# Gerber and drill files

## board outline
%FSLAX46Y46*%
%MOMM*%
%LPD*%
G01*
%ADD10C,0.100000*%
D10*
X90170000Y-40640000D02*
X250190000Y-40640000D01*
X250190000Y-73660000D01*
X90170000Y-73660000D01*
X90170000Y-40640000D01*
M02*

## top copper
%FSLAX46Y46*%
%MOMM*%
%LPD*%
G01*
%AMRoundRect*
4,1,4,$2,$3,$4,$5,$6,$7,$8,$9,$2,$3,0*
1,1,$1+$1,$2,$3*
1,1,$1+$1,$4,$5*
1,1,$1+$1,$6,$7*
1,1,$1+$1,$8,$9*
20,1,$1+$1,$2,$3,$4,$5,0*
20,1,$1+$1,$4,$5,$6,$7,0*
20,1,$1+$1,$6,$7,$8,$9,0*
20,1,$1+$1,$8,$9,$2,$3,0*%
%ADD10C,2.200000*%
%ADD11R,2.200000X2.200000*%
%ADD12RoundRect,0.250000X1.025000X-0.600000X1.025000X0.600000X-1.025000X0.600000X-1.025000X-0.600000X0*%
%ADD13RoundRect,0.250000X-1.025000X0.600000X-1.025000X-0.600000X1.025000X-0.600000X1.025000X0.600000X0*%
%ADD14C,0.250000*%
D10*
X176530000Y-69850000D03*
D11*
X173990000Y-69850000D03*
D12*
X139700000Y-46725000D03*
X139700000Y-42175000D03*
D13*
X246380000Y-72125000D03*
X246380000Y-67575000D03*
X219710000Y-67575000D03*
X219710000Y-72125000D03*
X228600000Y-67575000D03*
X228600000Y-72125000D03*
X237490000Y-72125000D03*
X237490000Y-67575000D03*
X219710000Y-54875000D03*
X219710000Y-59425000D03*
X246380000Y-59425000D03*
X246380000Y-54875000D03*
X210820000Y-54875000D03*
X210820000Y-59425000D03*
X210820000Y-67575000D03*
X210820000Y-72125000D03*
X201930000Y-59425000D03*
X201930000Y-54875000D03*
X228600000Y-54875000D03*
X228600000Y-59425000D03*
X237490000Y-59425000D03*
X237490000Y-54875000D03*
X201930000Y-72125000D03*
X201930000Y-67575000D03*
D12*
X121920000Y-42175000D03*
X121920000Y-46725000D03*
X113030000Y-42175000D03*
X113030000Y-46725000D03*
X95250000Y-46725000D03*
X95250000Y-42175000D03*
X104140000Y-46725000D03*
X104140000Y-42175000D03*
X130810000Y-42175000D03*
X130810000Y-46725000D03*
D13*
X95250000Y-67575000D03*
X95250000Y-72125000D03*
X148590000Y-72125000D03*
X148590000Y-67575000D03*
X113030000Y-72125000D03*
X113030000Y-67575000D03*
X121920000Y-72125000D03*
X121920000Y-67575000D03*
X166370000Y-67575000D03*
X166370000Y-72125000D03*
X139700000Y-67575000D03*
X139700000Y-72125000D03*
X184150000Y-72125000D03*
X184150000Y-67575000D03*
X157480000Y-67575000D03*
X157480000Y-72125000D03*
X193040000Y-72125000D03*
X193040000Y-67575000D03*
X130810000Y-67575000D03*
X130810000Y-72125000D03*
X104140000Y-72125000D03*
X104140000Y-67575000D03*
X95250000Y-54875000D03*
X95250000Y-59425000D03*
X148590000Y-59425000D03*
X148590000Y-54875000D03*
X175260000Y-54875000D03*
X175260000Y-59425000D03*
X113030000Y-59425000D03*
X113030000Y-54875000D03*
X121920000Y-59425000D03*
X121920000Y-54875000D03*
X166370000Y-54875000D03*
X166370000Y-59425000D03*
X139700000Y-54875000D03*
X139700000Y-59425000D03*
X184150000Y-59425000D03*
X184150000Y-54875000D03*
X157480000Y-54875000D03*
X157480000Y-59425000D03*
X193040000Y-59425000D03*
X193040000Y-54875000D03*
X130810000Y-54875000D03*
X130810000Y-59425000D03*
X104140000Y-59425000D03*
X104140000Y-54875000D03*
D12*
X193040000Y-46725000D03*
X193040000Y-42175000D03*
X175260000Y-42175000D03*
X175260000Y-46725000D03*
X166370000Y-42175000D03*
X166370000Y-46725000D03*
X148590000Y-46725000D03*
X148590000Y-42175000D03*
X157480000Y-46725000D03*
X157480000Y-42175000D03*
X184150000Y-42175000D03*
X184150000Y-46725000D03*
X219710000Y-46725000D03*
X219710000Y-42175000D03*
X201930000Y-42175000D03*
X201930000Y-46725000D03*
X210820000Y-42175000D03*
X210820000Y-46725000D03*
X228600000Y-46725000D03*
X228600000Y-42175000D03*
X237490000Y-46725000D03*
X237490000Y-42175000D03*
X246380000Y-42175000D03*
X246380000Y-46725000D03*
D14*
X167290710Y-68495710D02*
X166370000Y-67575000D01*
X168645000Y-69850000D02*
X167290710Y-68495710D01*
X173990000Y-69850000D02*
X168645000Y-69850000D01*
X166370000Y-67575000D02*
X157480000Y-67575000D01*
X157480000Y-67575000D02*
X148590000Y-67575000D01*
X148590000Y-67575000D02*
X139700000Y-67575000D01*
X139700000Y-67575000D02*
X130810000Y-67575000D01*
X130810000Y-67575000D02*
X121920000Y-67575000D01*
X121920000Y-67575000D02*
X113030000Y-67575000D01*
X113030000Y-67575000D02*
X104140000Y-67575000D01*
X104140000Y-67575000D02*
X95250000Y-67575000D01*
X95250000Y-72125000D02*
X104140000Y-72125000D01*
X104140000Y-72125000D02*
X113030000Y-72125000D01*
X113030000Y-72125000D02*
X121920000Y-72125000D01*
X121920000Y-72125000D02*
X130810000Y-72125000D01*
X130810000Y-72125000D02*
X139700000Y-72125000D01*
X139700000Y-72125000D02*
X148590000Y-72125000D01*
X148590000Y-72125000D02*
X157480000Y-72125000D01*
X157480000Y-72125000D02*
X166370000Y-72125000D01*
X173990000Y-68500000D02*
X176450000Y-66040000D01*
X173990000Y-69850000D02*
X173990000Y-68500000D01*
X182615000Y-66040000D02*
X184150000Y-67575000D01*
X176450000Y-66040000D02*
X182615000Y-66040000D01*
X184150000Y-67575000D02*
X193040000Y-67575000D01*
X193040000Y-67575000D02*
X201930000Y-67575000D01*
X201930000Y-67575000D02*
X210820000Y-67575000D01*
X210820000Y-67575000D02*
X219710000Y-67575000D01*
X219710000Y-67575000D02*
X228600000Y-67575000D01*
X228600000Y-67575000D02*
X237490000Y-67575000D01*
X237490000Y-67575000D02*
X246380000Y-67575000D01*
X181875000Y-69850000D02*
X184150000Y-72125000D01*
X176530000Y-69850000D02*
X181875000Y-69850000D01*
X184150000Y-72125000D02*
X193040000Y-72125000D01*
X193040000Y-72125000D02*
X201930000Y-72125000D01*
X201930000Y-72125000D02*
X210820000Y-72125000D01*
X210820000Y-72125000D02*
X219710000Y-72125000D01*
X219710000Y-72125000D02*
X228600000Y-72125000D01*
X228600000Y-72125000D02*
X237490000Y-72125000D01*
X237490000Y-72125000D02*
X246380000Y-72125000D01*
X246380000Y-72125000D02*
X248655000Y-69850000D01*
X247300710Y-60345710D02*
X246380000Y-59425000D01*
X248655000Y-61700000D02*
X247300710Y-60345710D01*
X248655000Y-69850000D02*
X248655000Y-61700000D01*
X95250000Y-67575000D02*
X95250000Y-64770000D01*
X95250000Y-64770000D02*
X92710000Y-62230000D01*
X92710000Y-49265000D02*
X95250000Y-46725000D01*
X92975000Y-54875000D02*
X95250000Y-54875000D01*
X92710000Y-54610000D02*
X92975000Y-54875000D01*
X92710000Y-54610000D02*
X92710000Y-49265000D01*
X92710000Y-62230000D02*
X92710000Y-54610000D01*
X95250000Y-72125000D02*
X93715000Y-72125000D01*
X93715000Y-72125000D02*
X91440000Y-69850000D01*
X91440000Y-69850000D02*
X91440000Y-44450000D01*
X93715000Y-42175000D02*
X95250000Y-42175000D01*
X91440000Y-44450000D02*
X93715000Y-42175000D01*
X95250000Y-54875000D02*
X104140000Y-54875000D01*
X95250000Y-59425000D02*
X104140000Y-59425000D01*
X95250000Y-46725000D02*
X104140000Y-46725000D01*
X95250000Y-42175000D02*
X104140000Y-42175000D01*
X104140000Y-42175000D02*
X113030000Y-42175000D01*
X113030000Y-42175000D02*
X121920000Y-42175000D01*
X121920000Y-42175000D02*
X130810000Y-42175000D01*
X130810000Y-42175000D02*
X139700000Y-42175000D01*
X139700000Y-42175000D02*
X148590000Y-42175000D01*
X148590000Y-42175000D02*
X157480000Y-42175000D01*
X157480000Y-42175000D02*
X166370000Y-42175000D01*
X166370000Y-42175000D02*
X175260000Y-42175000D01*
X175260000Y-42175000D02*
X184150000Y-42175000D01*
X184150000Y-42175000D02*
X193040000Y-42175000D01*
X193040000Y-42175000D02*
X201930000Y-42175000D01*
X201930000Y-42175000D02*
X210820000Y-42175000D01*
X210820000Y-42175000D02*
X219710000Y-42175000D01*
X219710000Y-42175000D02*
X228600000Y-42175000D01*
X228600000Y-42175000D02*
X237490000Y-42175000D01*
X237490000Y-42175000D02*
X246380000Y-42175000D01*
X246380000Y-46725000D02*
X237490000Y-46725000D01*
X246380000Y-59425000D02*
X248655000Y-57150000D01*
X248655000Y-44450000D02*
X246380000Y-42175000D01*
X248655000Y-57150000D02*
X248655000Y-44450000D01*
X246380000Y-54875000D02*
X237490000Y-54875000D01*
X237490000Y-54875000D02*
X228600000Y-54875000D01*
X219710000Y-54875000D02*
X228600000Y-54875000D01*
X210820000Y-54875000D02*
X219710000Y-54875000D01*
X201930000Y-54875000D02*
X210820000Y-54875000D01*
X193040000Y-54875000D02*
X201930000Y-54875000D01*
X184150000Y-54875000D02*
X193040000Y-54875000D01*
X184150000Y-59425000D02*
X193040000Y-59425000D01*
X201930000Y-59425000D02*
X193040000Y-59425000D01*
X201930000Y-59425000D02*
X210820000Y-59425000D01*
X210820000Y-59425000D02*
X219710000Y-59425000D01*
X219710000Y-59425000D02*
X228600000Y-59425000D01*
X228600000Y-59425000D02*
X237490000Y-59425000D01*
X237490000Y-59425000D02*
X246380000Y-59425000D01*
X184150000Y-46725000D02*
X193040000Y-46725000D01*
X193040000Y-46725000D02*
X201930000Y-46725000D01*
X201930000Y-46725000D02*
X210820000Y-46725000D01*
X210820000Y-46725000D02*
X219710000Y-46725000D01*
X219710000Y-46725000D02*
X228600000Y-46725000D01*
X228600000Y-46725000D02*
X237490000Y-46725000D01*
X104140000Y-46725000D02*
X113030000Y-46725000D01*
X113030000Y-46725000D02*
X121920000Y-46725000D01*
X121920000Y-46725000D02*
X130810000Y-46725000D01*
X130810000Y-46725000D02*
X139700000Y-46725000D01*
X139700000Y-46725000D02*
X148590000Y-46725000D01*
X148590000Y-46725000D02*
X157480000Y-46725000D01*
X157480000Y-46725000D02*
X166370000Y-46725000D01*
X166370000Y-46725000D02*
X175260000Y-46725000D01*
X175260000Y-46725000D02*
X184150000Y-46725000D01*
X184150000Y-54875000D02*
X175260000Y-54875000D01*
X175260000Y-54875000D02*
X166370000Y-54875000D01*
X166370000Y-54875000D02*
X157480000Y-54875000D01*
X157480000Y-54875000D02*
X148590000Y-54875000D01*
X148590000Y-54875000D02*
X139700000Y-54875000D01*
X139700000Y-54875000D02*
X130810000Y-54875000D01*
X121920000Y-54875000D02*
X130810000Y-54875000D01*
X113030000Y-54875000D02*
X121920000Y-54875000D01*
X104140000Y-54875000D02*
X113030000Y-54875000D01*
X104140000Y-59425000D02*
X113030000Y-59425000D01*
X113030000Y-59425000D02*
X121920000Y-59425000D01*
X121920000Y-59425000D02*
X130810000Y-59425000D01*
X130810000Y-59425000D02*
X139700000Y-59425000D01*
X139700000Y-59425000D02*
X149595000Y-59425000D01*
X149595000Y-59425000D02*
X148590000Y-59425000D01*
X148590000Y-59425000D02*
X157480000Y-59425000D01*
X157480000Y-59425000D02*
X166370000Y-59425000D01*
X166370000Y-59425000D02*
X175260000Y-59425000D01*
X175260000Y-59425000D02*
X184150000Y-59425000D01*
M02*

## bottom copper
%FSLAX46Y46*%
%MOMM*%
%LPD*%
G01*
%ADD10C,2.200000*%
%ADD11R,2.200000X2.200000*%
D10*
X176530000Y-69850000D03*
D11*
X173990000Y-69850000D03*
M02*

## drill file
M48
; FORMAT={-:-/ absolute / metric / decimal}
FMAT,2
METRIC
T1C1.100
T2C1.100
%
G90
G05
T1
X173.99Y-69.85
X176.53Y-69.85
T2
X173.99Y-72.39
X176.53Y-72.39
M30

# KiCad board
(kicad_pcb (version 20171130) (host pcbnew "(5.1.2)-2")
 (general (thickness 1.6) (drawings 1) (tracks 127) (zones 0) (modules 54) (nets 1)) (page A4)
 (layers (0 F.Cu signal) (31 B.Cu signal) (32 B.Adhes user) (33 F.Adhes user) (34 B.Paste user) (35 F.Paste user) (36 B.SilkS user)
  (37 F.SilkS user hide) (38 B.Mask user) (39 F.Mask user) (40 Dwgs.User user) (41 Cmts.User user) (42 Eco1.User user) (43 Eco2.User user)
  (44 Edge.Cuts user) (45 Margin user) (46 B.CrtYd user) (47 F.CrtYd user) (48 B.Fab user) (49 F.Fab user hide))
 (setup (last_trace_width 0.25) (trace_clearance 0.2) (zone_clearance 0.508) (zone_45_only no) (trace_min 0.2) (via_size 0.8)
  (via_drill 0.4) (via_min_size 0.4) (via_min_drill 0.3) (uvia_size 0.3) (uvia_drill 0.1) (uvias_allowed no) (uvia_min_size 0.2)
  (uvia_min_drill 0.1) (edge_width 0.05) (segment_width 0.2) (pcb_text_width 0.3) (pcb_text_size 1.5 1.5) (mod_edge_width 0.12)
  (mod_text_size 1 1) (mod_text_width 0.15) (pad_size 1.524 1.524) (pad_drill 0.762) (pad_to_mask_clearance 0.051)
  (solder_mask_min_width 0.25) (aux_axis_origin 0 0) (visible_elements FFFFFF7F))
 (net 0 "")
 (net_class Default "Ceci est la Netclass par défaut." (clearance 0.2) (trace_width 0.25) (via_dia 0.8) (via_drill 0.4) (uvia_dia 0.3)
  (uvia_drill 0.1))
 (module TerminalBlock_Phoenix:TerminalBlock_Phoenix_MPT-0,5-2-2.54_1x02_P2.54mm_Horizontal (layer F.Cu) (at 173.99 69.85)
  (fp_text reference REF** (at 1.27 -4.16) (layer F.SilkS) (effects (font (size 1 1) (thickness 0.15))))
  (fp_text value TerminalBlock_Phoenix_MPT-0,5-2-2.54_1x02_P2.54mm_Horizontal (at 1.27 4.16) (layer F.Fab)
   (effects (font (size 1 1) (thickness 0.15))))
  (pad "" np_thru_hole circle (at 2.54 2.54) (size 1.1 1.1) (drill 1.1) (layers *.Cu *.Mask))
  (pad 2 thru_hole circle (at 2.54 0) (size 2.2 2.2) (drill 1.1) (layers *.Cu *.Mask))
  (pad "" np_thru_hole circle (at 0 2.54) (size 1.1 1.1) (drill 1.1) (layers *.Cu *.Mask))
  (pad 1 thru_hole rect (at 0 0) (size 2.2 2.2) (drill 1.1) (layers *.Cu *.Mask)))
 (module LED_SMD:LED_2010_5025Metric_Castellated (layer F.Cu) (at 139.7 44.45 90)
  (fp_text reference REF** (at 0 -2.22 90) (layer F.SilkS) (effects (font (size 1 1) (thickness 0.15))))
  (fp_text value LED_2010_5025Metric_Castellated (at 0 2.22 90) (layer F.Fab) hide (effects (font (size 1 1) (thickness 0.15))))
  (pad 1 smd roundrect (at -2.275 0 90) (size 1.7 2.55) (layers F.Cu F.Paste F.Mask) (roundrect_rratio 0.147059))
  (pad 2 smd roundrect (at 2.275 0 90) (size 1.7 2.55) (layers F.Cu F.Paste F.Mask) (roundrect_rratio 0.147059)))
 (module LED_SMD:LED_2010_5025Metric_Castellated (layer F.Cu) (at 246.38 69.85 270)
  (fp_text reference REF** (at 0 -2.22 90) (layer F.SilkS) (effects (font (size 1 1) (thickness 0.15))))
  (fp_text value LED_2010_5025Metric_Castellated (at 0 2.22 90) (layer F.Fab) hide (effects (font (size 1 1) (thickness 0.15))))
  (pad 2 smd roundrect (at 2.275 0 270) (size 1.7 2.55) (layers F.Cu F.Paste F.Mask) (roundrect_rratio 0.147059))
  (pad 1 smd roundrect (at -2.275 0 270) (size 1.7 2.55) (layers F.Cu F.Paste F.Mask) (roundrect_rratio 0.147059)))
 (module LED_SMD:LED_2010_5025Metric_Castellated (layer F.Cu) (at 219.71 69.85 270)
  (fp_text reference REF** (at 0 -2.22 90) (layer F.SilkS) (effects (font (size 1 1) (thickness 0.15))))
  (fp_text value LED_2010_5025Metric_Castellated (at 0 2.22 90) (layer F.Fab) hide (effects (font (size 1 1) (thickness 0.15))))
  (pad 1 smd roundrect (at -2.275 0 270) (size 1.7 2.55) (layers F.Cu F.Paste F.Mask) (roundrect_rratio 0.147059))
  (pad 2 smd roundrect (at 2.275 0 270) (size 1.7 2.55) (layers F.Cu F.Paste F.Mask) (roundrect_rratio 0.147059)))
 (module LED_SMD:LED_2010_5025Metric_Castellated (layer F.Cu) (at 228.6 69.85 270)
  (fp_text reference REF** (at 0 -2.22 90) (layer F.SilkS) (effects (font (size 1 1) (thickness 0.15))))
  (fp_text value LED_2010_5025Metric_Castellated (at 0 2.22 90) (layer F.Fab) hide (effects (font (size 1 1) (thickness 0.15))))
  (pad 1 smd roundrect (at -2.275 0 270) (size 1.7 2.55) (layers F.Cu F.Paste F.Mask) (roundrect_rratio 0.147059))
  (pad 2 smd roundrect (at 2.275 0 270) (size 1.7 2.55) (layers F.Cu F.Paste F.Mask) (roundrect_rratio 0.147059)))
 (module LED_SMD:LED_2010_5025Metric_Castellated (layer F.Cu) (at 237.49 69.85 270)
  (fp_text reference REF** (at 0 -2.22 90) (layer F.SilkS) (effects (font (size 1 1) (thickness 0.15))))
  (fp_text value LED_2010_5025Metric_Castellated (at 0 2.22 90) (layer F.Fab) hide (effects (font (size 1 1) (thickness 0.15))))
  (pad 2 smd roundrect (at 2.275 0 270) (size 1.7 2.55) (layers F.Cu F.Paste F.Mask) (roundrect_rratio 0.147059))
  (pad 1 smd roundrect (at -2.275 0 270) (size 1.7 2.55) (layers F.Cu F.Paste F.Mask) (roundrect_rratio 0.147059)))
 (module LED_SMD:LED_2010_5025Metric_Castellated (layer F.Cu) (at 219.71 57.15 270)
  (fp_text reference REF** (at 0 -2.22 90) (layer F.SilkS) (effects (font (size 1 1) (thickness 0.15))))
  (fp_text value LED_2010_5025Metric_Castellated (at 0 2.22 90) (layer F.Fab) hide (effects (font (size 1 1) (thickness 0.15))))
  (pad 1 smd roundrect (at -2.275 0 270) (size 1.7 2.55) (layers F.Cu F.Paste F.Mask) (roundrect_rratio 0.147059))
  (pad 2 smd roundrect (at 2.275 0 270) (size 1.7 2.55) (layers F.Cu F.Paste F.Mask) (roundrect_rratio 0.147059)))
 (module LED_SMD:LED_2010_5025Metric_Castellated (layer F.Cu) (at 246.38 57.15 270)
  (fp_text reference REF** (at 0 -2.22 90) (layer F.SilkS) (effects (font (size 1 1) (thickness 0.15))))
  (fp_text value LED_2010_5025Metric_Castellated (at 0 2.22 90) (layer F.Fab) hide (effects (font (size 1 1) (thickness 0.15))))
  (pad 2 smd roundrect (at 2.275 0 270) (size 1.7 2.55) (layers F.Cu F.Paste F.Mask) (roundrect_rratio 0.147059))
  (pad 1 smd roundrect (at -2.275 0 270) (size 1.7 2.55) (layers F.Cu F.Paste F.Mask) (roundrect_rratio 0.147059)))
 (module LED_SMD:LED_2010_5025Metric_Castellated (layer F.Cu) (at 210.82 57.15 270)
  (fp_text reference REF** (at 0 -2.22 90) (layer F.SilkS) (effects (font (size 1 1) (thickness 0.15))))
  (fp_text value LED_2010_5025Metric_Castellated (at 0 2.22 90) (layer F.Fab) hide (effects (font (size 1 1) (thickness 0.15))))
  (pad 1 smd roundrect (at -2.275 0 270) (size 1.7 2.55) (layers F.Cu F.Paste F.Mask) (roundrect_rratio 0.147059))
  (pad 2 smd roundrect (at 2.275 0 270) (size 1.7 2.55) (layers F.Cu F.Paste F.Mask) (roundrect_rratio 0.147059)))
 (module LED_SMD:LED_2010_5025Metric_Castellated (layer F.Cu) (at 210.82 69.85 270)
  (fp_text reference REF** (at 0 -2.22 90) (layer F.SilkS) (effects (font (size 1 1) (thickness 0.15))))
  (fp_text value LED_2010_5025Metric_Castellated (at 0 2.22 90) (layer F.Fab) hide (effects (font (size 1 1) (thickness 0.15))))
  (pad 1 smd roundrect (at -2.275 0 270) (size 1.7 2.55) (layers F.Cu F.Paste F.Mask) (roundrect_rratio 0.147059))
  (pad 2 smd roundrect (at 2.275 0 270) (size 1.7 2.55) (layers F.Cu F.Paste F.Mask) (roundrect_rratio 0.147059)))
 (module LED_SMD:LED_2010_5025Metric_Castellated (layer F.Cu) (at 201.93 57.15 270)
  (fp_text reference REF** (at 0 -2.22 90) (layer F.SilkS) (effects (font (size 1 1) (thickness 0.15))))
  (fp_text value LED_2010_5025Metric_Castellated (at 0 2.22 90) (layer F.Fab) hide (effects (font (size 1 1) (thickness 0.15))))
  (pad 2 smd roundrect (at 2.275 0 270) (size 1.7 2.55) (layers F.Cu F.Paste F.Mask) (roundrect_rratio 0.147059))
  (pad 1 smd roundrect (at -2.275 0 270) (size 1.7 2.55) (layers F.Cu F.Paste F.Mask) (roundrect_rratio 0.147059)))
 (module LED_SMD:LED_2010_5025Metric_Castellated (layer F.Cu) (at 228.6 57.15 270)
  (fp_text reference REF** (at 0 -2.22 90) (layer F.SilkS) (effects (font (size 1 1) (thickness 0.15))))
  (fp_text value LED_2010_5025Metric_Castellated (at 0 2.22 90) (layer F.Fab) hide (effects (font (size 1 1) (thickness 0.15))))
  (pad 1 smd roundrect (at -2.275 0 270) (size 1.7 2.55) (layers F.Cu F.Paste F.Mask) (roundrect_rratio 0.147059))
  (pad 2 smd roundrect (at 2.275 0 270) (size 1.7 2.55) (layers F.Cu F.Paste F.Mask) (roundrect_rratio 0.147059)))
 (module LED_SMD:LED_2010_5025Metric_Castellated (layer F.Cu) (at 237.49 57.15 270)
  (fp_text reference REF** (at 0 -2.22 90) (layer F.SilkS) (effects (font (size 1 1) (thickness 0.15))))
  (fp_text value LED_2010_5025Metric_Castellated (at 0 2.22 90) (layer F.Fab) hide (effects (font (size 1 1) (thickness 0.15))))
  (pad 2 smd roundrect (at 2.275 0 270) (size 1.7 2.55) (layers F.Cu F.Paste F.Mask) (roundrect_rratio 0.147059))
  (pad 1 smd roundrect (at -2.275 0 270) (size 1.7 2.55) (layers F.Cu F.Paste F.Mask) (roundrect_rratio 0.147059)))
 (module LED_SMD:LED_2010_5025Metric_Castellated (layer F.Cu) (at 201.93 69.85 270)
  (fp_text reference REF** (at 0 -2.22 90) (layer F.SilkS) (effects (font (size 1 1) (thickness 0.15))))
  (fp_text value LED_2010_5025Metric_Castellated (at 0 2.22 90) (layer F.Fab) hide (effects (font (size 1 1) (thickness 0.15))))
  (pad 2 smd roundrect (at 2.275 0 270) (size 1.7 2.55) (layers F.Cu F.Paste F.Mask) (roundrect_rratio 0.147059))
  (pad 1 smd roundrect (at -2.275 0 270) (size 1.7 2.55) (layers F.Cu F.Paste F.Mask) (roundrect_rratio 0.147059)))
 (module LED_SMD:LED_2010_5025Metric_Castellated (layer F.Cu) (at 121.92 44.45 90)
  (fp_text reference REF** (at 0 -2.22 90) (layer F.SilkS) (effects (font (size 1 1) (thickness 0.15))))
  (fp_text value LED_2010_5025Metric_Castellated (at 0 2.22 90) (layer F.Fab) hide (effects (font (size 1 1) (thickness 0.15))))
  (pad 2 smd roundrect (at 2.275 0 90) (size 1.7 2.55) (layers F.Cu F.Paste F.Mask) (roundrect_rratio 0.147059))
  (pad 1 smd roundrect (at -2.275 0 90) (size 1.7 2.55) (layers F.Cu F.Paste F.Mask) (roundrect_rratio 0.147059)))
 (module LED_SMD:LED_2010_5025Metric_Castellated (layer F.Cu) (at 113.03 44.45 90)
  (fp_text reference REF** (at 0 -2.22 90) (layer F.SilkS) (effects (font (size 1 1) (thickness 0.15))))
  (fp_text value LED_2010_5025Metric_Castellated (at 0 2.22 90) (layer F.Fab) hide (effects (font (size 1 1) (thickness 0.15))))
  (pad 2 smd roundrect (at 2.275 0 90) (size 1.7 2.55) (layers F.Cu F.Paste F.Mask) (roundrect_rratio 0.147059))
  (pad 1 smd roundrect (at -2.275 0 90) (size 1.7 2.55) (layers F.Cu F.Paste F.Mask) (roundrect_rratio 0.147059)))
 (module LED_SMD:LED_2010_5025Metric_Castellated (layer F.Cu) (at 95.25 44.45 90)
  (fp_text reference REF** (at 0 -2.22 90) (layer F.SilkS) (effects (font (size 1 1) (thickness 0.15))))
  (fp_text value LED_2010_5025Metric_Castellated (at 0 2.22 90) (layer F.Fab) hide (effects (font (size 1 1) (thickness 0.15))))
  (pad 1 smd roundrect (at -2.275 0 90) (size 1.7 2.55) (layers F.Cu F.Paste F.Mask) (roundrect_rratio 0.147059))
  (pad 2 smd roundrect (at 2.275 0 90) (size 1.7 2.55) (layers F.Cu F.Paste F.Mask) (roundrect_rratio 0.147059)))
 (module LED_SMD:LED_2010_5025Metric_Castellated (layer F.Cu) (at 104.14 44.45 90)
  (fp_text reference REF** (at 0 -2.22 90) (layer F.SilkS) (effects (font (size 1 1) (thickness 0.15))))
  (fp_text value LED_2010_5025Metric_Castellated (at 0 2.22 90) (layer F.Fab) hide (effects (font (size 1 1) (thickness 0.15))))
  (pad 1 smd roundrect (at -2.275 0 90) (size 1.7 2.55) (layers F.Cu F.Paste F.Mask) (roundrect_rratio 0.147059))
  (pad 2 smd roundrect (at 2.275 0 90) (size 1.7 2.55) (layers F.Cu F.Paste F.Mask) (roundrect_rratio 0.147059)))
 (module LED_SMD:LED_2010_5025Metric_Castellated (layer F.Cu) (at 130.81 44.45 90)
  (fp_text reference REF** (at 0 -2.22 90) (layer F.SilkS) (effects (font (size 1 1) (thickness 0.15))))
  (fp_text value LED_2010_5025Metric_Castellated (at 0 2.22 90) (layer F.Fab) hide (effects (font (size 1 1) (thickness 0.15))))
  (pad 2 smd roundrect (at 2.275 0 90) (size 1.7 2.55) (layers F.Cu F.Paste F.Mask) (roundrect_rratio 0.147059))
  (pad 1 smd roundrect (at -2.275 0 90) (size 1.7 2.55) (layers F.Cu F.Paste F.Mask) (roundrect_rratio 0.147059)))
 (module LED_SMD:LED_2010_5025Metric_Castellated (layer F.Cu) (at 95.25 69.85 270)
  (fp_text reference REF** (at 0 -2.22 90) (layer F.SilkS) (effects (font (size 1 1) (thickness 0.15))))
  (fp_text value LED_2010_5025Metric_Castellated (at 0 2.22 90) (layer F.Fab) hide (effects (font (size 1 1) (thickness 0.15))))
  (pad 1 smd roundrect (at -2.275 0 270) (size 1.7 2.55) (layers F.Cu F.Paste F.Mask) (roundrect_rratio 0.147059))
  (pad 2 smd roundrect (at 2.275 0 270) (size 1.7 2.55) (layers F.Cu F.Paste F.Mask) (roundrect_rratio 0.147059)))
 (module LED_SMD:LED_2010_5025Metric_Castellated (layer F.Cu) (at 148.59 69.85 270)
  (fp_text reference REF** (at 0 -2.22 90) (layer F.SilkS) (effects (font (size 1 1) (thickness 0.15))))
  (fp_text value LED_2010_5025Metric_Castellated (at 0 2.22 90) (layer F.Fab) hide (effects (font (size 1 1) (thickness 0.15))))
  (pad 2 smd roundrect (at 2.275 0 270) (size 1.7 2.55) (layers F.Cu F.Paste F.Mask) (roundrect_rratio 0.147059))
  (pad 1 smd roundrect (at -2.275 0 270) (size 1.7 2.55) (layers F.Cu F.Paste F.Mask) (roundrect_rratio 0.147059)))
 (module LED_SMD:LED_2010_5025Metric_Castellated (layer F.Cu) (at 113.03 69.85 270)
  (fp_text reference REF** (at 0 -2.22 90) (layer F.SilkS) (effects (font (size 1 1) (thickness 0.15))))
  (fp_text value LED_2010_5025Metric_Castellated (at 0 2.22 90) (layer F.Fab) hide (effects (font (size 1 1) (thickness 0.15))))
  (pad 2 smd roundrect (at 2.275 0 270) (size 1.7 2.55) (layers F.Cu F.Paste F.Mask) (roundrect_rratio 0.147059))
  (pad 1 smd roundrect (at -2.275 0 270) (size 1.7 2.55) (layers F.Cu F.Paste F.Mask) (roundrect_rratio 0.147059)))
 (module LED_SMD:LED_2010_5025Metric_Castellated (layer F.Cu) (at 121.92 69.85 270)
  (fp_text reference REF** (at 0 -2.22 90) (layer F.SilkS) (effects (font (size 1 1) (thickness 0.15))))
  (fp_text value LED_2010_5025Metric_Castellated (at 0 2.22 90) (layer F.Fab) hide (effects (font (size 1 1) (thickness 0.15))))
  (pad 2 smd roundrect (at 2.275 0 270) (size 1.7 2.55) (layers F.Cu F.Paste F.Mask) (roundrect_rratio 0.147059))
  (pad 1 smd roundrect (at -2.275 0 270) (size 1.7 2.55) (layers F.Cu F.Paste F.Mask) (roundrect_rratio 0.147059)))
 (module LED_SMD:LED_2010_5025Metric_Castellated (layer F.Cu) (at 166.37 69.85 270)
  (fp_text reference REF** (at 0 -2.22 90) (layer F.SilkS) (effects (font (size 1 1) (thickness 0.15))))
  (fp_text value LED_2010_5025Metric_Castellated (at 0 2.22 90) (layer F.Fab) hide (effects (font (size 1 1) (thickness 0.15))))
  (pad 1 smd roundrect (at -2.275 0 270) (size 1.7 2.55) (layers F.Cu F.Paste F.Mask) (roundrect_rratio 0.147059))
  (pad 2 smd roundrect (at 2.275 0 270) (size 1.7 2.55) (layers F.Cu F.Paste F.Mask) (roundrect_rratio 0.147059)))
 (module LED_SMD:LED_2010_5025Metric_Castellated (layer F.Cu) (at 139.7 69.85 270)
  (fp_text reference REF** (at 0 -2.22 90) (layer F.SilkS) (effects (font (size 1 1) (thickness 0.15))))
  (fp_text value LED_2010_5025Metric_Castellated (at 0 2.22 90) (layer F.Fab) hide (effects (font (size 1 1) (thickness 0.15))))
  (pad 1 smd roundrect (at -2.275 0 270) (size 1.7 2.55) (layers F.Cu F.Paste F.Mask) (roundrect_rratio 0.147059))
  (pad 2 smd roundrect (at 2.275 0 270) (size 1.7 2.55) (layers F.Cu F.Paste F.Mask) (roundrect_rratio 0.147059)))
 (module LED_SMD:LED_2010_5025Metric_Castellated (layer F.Cu) (at 184.15 69.85 270)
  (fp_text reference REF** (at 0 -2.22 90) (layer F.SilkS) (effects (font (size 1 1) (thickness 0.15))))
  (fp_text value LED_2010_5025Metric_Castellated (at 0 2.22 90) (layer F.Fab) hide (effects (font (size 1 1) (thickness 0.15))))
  (pad 2 smd roundrect (at 2.275 0 270) (size 1.7 2.55) (layers F.Cu F.Paste F.Mask) (roundrect_rratio 0.147059))
  (pad 1 smd roundrect (at -2.275 0 270) (size 1.7 2.55) (layers F.Cu F.Paste F.Mask) (roundrect_rratio 0.147059)))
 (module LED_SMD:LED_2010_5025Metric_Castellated (layer F.Cu) (at 157.48 69.85 270)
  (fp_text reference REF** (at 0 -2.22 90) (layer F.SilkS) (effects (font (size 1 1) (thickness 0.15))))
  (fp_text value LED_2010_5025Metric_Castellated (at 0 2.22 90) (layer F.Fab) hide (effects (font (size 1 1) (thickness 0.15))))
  (pad 1 smd roundrect (at -2.275 0 270) (size 1.7 2.55) (layers F.Cu F.Paste F.Mask) (roundrect_rratio 0.147059))
  (pad 2 smd roundrect (at 2.275 0 270) (size 1.7 2.55) (layers F.Cu F.Paste F.Mask) (roundrect_rratio 0.147059)))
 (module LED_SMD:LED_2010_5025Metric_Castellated (layer F.Cu) (at 193.04 69.85 270)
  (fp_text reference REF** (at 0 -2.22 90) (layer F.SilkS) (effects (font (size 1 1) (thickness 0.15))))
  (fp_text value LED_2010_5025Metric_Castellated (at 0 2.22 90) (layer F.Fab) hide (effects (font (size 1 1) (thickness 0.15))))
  (pad 2 smd roundrect (at 2.275 0 270) (size 1.7 2.55) (layers F.Cu F.Paste F.Mask) (roundrect_rratio 0.147059))
  (pad 1 smd roundrect (at -2.275 0 270) (size 1.7 2.55) (layers F.Cu F.Paste F.Mask) (roundrect_rratio 0.147059)))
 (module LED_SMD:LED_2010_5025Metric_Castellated (layer F.Cu) (at 130.81 69.85 270)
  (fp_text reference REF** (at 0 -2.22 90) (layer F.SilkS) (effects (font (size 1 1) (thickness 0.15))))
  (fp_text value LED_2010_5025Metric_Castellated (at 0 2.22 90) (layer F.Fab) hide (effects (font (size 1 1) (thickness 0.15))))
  (pad 1 smd roundrect (at -2.275 0 270) (size 1.7 2.55) (layers F.Cu F.Paste F.Mask) (roundrect_rratio 0.147059))
  (pad 2 smd roundrect (at 2.275 0 270) (size 1.7 2.55) (layers F.Cu F.Paste F.Mask) (roundrect_rratio 0.147059)))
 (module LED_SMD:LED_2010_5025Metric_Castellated (layer F.Cu) (at 104.14 69.85 270)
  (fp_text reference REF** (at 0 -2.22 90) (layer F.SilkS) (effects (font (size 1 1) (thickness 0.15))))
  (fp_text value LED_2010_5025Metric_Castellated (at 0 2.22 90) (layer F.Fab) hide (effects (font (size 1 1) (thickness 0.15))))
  (pad 2 smd roundrect (at 2.275 0 270) (size 1.7 2.55) (layers F.Cu F.Paste F.Mask) (roundrect_rratio 0.147059))
  (pad 1 smd roundrect (at -2.275 0 270) (size 1.7 2.55) (layers F.Cu F.Paste F.Mask) (roundrect_rratio 0.147059)))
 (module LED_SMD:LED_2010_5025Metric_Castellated (layer F.Cu) (at 95.25 57.15 270)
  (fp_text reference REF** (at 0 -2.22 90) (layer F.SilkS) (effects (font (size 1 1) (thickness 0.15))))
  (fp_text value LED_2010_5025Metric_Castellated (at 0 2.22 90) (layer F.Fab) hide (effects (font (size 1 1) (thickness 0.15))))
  (pad 1 smd roundrect (at -2.275 0 270) (size 1.7 2.55) (layers F.Cu F.Paste F.Mask) (roundrect_rratio 0.147059))
  (pad 2 smd roundrect (at 2.275 0 270) (size 1.7 2.55) (layers F.Cu F.Paste F.Mask) (roundrect_rratio 0.147059)))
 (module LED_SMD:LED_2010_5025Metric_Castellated (layer F.Cu) (at 148.59 57.15 270)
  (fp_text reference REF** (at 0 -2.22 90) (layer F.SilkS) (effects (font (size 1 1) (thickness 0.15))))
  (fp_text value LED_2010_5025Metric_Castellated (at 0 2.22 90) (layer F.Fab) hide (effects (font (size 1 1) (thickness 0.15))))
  (pad 2 smd roundrect (at 2.275 0 270) (size 1.7 2.55) (layers F.Cu F.Paste F.Mask) (roundrect_rratio 0.147059))
  (pad 1 smd roundrect (at -2.275 0 270) (size 1.7 2.55) (layers F.Cu F.Paste F.Mask) (roundrect_rratio 0.147059)))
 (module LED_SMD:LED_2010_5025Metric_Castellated (layer F.Cu) (at 175.26 57.15 270)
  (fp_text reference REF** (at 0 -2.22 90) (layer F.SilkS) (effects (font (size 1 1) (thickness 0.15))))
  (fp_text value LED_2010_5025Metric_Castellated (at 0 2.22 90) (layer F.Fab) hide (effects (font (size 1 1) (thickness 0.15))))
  (pad 1 smd roundrect (at -2.275 0 270) (size 1.7 2.55) (layers F.Cu F.Paste F.Mask) (roundrect_rratio 0.147059))
  (pad 2 smd roundrect (at 2.275 0 270) (size 1.7 2.55) (layers F.Cu F.Paste F.Mask) (roundrect_rratio 0.147059)))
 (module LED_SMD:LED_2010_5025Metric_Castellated (layer F.Cu) (at 113.03 57.15 270)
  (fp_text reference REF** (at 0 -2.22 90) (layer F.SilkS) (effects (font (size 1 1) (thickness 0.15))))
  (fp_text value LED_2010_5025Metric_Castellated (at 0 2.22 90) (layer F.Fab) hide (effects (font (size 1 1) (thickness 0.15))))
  (pad 2 smd roundrect (at 2.275 0 270) (size 1.7 2.55) (layers F.Cu F.Paste F.Mask) (roundrect_rratio 0.147059))
  (pad 1 smd roundrect (at -2.275 0 270) (size 1.7 2.55) (layers F.Cu F.Paste F.Mask) (roundrect_rratio 0.147059)))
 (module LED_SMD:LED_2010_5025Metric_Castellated (layer F.Cu) (at 121.92 57.15 270)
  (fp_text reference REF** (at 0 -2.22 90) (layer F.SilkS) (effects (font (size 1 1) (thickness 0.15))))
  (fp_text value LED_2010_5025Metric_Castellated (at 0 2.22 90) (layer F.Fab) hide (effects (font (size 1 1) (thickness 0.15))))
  (pad 2 smd roundrect (at 2.275 0 270) (size 1.7 2.55) (layers F.Cu F.Paste F.Mask) (roundrect_rratio 0.147059))
  (pad 1 smd roundrect (at -2.275 0 270) (size 1.7 2.55) (layers F.Cu F.Paste F.Mask) (roundrect_rratio 0.147059)))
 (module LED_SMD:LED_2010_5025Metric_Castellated (layer F.Cu) (at 166.37 57.15 270)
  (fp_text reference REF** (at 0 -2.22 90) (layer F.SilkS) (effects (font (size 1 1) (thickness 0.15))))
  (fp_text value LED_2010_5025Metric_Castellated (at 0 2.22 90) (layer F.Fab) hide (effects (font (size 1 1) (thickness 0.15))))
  (pad 1 smd roundrect (at -2.275 0 270) (size 1.7 2.55) (layers F.Cu F.Paste F.Mask) (roundrect_rratio 0.147059))
  (pad 2 smd roundrect (at 2.275 0 270) (size 1.7 2.55) (layers F.Cu F.Paste F.Mask) (roundrect_rratio 0.147059)))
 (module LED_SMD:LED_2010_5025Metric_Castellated (layer F.Cu) (at 139.7 57.15 270)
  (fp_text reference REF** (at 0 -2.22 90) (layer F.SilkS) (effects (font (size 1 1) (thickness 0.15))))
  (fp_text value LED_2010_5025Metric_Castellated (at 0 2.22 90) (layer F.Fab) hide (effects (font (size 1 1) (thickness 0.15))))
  (pad 1 smd roundrect (at -2.275 0 270) (size 1.7 2.55) (layers F.Cu F.Paste F.Mask) (roundrect_rratio 0.147059))
  (pad 2 smd roundrect (at 2.275 0 270) (size 1.7 2.55) (layers F.Cu F.Paste F.Mask) (roundrect_rratio 0.147059)))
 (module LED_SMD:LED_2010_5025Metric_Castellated (layer F.Cu) (at 184.15 57.15 270)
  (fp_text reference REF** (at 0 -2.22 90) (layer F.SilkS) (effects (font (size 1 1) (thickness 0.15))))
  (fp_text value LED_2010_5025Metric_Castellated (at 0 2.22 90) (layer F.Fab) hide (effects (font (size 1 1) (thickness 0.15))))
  (pad 2 smd roundrect (at 2.275 0 270) (size 1.7 2.55) (layers F.Cu F.Paste F.Mask) (roundrect_rratio 0.147059))
  (pad 1 smd roundrect (at -2.275 0 270) (size 1.7 2.55) (layers F.Cu F.Paste F.Mask) (roundrect_rratio 0.147059)))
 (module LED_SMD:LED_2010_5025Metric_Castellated (layer F.Cu) (at 157.48 57.15 270)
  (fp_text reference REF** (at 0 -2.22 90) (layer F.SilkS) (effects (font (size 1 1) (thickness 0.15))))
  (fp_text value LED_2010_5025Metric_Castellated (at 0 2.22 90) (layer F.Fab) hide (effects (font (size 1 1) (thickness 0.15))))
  (pad 1 smd roundrect (at -2.275 0 270) (size 1.7 2.55) (layers F.Cu F.Paste F.Mask) (roundrect_rratio 0.147059))
  (pad 2 smd roundrect (at 2.275 0 270) (size 1.7 2.55) (layers F.Cu F.Paste F.Mask) (roundrect_rratio 0.147059)))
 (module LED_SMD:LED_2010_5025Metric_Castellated (layer F.Cu) (at 193.04 57.15 270)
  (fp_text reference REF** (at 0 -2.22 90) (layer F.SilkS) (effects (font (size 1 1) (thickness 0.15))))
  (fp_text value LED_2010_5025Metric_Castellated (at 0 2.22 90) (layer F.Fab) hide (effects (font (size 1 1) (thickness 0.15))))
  (pad 2 smd roundrect (at 2.275 0 270) (size 1.7 2.55) (layers F.Cu F.Paste F.Mask) (roundrect_rratio 0.147059))
  (pad 1 smd roundrect (at -2.275 0 270) (size 1.7 2.55) (layers F.Cu F.Paste F.Mask) (roundrect_rratio 0.147059)))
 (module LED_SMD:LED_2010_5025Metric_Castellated (layer F.Cu) (at 130.81 57.15 270)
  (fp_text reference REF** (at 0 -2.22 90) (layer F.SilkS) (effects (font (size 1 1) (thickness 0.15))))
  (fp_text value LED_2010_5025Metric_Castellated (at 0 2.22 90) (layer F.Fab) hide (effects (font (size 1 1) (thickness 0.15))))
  (pad 1 smd roundrect (at -2.275 0 270) (size 1.7 2.55) (layers F.Cu F.Paste F.Mask) (roundrect_rratio 0.147059))
  (pad 2 smd roundrect (at 2.275 0 270) (size 1.7 2.55) (layers F.Cu F.Paste F.Mask) (roundrect_rratio 0.147059)))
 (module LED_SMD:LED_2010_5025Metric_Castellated (layer F.Cu) (at 104.14 57.15 270)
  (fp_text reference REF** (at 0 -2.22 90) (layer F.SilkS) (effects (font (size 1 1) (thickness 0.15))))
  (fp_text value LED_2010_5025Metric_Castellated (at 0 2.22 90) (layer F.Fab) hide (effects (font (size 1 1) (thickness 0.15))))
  (pad 2 smd roundrect (at 2.275 0 270) (size 1.7 2.55) (layers F.Cu F.Paste F.Mask) (roundrect_rratio 0.147059))
  (pad 1 smd roundrect (at -2.275 0 270) (size 1.7 2.55) (layers F.Cu F.Paste F.Mask) (roundrect_rratio 0.147059)))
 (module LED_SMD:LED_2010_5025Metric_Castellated (layer F.Cu) (at 193.04 44.45 90)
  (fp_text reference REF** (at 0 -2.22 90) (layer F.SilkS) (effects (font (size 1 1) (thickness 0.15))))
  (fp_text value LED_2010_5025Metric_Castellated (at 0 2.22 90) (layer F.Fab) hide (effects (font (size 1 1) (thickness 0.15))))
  (pad 1 smd roundrect (at -2.275 0 90) (size 1.7 2.55) (layers F.Cu F.Paste F.Mask) (roundrect_rratio 0.147059))
  (pad 2 smd roundrect (at 2.275 0 90) (size 1.7 2.55) (layers F.Cu F.Paste F.Mask) (roundrect_rratio 0.147059)))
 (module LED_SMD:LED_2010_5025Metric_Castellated (layer F.Cu) (at 175.26 44.45 90)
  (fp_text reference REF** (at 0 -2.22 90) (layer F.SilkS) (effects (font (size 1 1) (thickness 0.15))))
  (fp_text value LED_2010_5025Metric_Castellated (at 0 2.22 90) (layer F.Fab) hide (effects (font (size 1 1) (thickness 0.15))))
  (pad 2 smd roundrect (at 2.275 0 90) (size 1.7 2.55) (layers F.Cu F.Paste F.Mask) (roundrect_rratio 0.147059))
  (pad 1 smd roundrect (at -2.275 0 90) (size 1.7 2.55) (layers F.Cu F.Paste F.Mask) (roundrect_rratio 0.147059)))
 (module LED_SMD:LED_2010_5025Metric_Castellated (layer F.Cu) (at 166.37 44.45 90)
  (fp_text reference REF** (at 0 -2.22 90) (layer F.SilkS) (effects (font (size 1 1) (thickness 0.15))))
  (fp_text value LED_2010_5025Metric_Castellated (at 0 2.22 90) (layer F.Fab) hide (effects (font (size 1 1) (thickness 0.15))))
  (pad 2 smd roundrect (at 2.275 0 90) (size 1.7 2.55) (layers F.Cu F.Paste F.Mask) (roundrect_rratio 0.147059))
  (pad 1 smd roundrect (at -2.275 0 90) (size 1.7 2.55) (layers F.Cu F.Paste F.Mask) (roundrect_rratio 0.147059)))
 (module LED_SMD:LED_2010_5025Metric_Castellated (layer F.Cu) (at 148.59 44.45 90)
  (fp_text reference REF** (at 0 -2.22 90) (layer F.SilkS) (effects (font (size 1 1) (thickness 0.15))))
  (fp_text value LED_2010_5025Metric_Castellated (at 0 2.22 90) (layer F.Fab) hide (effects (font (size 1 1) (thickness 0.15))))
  (pad 1 smd roundrect (at -2.275 0 90) (size 1.7 2.55) (layers F.Cu F.Paste F.Mask) (roundrect_rratio 0.147059))
  (pad 2 smd roundrect (at 2.275 0 90) (size 1.7 2.55) (layers F.Cu F.Paste F.Mask) (roundrect_rratio 0.147059)))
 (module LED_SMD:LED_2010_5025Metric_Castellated (layer F.Cu) (at 157.48 44.45 90)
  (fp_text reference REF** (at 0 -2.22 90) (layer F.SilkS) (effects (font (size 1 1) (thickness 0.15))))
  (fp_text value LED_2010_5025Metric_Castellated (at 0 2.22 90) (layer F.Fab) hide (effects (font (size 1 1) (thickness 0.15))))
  (pad 1 smd roundrect (at -2.275 0 90) (size 1.7 2.55) (layers F.Cu F.Paste F.Mask) (roundrect_rratio 0.147059))
  (pad 2 smd roundrect (at 2.275 0 90) (size 1.7 2.55) (layers F.Cu F.Paste F.Mask) (roundrect_rratio 0.147059)))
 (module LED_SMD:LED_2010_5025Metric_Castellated (layer F.Cu) (at 184.15 44.45 90)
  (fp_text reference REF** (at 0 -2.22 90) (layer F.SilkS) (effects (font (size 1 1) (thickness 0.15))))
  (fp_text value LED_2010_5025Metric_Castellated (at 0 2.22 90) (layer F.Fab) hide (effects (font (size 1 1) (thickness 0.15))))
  (pad 2 smd roundrect (at 2.275 0 90) (size 1.7 2.55) (layers F.Cu F.Paste F.Mask) (roundrect_rratio 0.147059))
  (pad 1 smd roundrect (at -2.275 0 90) (size 1.7 2.55) (layers F.Cu F.Paste F.Mask) (roundrect_rratio 0.147059)))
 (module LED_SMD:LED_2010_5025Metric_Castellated (layer F.Cu) (at 219.71 44.45 90)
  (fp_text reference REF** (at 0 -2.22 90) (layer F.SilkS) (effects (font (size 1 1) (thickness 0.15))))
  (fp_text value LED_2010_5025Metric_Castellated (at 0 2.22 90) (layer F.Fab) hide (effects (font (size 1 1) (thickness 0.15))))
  (pad 1 smd roundrect (at -2.275 0 90) (size 1.7 2.55) (layers F.Cu F.Paste F.Mask) (roundrect_rratio 0.147059))
  (pad 2 smd roundrect (at 2.275 0 90) (size 1.7 2.55) (layers F.Cu F.Paste F.Mask) (roundrect_rratio 0.147059)))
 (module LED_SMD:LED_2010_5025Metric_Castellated (layer F.Cu) (at 201.93 44.45 90)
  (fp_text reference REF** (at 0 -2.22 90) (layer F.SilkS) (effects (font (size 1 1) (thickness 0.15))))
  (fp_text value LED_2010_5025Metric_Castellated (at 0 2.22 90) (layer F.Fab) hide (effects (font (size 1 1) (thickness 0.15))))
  (pad 2 smd roundrect (at 2.275 0 90) (size 1.7 2.55) (layers F.Cu F.Paste F.Mask) (roundrect_rratio 0.147059))
  (pad 1 smd roundrect (at -2.275 0 90) (size 1.7 2.55) (layers F.Cu F.Paste F.Mask) (roundrect_rratio 0.147059)))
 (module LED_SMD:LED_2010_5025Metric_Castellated (layer F.Cu) (at 210.82 44.45 90)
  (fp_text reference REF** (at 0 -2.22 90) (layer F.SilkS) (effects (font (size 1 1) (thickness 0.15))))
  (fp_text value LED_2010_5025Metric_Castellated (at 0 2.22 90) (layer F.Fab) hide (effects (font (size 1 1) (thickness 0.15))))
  (pad 2 smd roundrect (at 2.275 0 90) (size 1.7 2.55) (layers F.Cu F.Paste F.Mask) (roundrect_rratio 0.147059))
  (pad 1 smd roundrect (at -2.275 0 90) (size 1.7 2.55) (layers F.Cu F.Paste F.Mask) (roundrect_rratio 0.147059)))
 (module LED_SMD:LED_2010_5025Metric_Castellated (layer F.Cu) (at 228.6 44.45 90)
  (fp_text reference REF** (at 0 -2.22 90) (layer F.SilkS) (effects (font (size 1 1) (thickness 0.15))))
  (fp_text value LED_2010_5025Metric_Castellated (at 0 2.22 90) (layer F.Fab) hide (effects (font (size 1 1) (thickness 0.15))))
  (pad 1 smd roundrect (at -2.275 0 90) (size 1.7 2.55) (layers F.Cu F.Paste F.Mask) (roundrect_rratio 0.147059))
  (pad 2 smd roundrect (at 2.275 0 90) (size 1.7 2.55) (layers F.Cu F.Paste F.Mask) (roundrect_rratio 0.147059)))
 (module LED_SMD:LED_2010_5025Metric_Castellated (layer F.Cu) (at 237.49 44.45 90)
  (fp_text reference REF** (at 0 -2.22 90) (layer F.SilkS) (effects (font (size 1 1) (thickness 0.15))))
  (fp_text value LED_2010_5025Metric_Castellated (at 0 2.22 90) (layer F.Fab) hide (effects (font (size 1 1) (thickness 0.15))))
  (pad 1 smd roundrect (at -2.275 0 90) (size 1.7 2.55) (layers F.Cu F.Paste F.Mask) (roundrect_rratio 0.147059))
  (pad 2 smd roundrect (at 2.275 0 90) (size 1.7 2.55) (layers F.Cu F.Paste F.Mask) (roundrect_rratio 0.147059)))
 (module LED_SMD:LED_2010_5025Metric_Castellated (layer F.Cu) (at 246.38 44.45 90)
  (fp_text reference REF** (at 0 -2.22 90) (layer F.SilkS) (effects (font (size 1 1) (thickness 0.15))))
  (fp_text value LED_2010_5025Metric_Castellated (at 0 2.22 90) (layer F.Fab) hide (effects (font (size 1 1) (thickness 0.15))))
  (pad 2 smd roundrect (at 2.275 0 90) (size 1.7 2.55) (layers F.Cu F.Paste F.Mask) (roundrect_rratio 0.147059))
  (pad 1 smd roundrect (at -2.275 0 90) (size 1.7 2.55) (layers F.Cu F.Paste F.Mask) (roundrect_rratio 0.147059)))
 (gr_poly (pts (xy 90.17 40.64) (xy 250.19 40.64) (xy 250.19 73.66) (xy 90.17 73.66)) (layer Edge.Cuts) (width 0.1))
 (segment (start 167.29071 68.49571) (end 166.37 67.575) (width 0.25) (layer F.Cu) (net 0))
 (segment (start 168.645 69.85) (end 167.29071 68.49571) (width 0.25) (layer F.Cu) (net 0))
 (segment (start 173.99 69.85) (end 168.645 69.85) (width 0.25) (layer F.Cu) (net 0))
 (segment (start 166.37 67.575) (end 157.48 67.575) (width 0.25) (layer F.Cu) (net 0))
 (segment (start 157.48 67.575) (end 148.59 67.575) (width 0.25) (layer F.Cu) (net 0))
 (segment (start 148.59 67.575) (end 139.7 67.575) (width 0.25) (layer F.Cu) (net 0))
 (segment (start 139.7 67.575) (end 130.81 67.575) (width 0.25) (layer F.Cu) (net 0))
 (segment (start 130.81 67.575) (end 121.92 67.575) (width 0.25) (layer F.Cu) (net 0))
 (segment (start 121.92 67.575) (end 113.03 67.575) (width 0.25) (layer F.Cu) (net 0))
 (segment (start 113.03 67.575) (end 104.14 67.575) (width 0.25) (layer F.Cu) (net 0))
 (segment (start 104.14 67.575) (end 95.25 67.575) (width 0.25) (layer F.Cu) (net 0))
 (segment (start 95.25 72.125) (end 104.14 72.125) (width 0.25) (layer F.Cu) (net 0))
 (segment (start 104.14 72.125) (end 113.03 72.125) (width 0.25) (layer F.Cu) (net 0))
 (segment (start 113.03 72.125) (end 121.92 72.125) (width 0.25) (layer F.Cu) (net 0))
 (segment (start 121.92 72.125) (end 130.81 72.125) (width 0.25) (layer F.Cu) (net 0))
 (segment (start 130.81 72.125) (end 139.7 72.125) (width 0.25) (layer F.Cu) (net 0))
 (segment (start 139.7 72.125) (end 148.59 72.125) (width 0.25) (layer F.Cu) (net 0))
 (segment (start 148.59 72.125) (end 157.48 72.125) (width 0.25) (layer F.Cu) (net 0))
 (segment (start 157.48 72.125) (end 166.37 72.125) (width 0.25) (layer F.Cu) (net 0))
 (segment (start 173.99 68.5) (end 176.45 66.04) (width 0.25) (layer F.Cu) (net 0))
 (segment (start 173.99 69.85) (end 173.99 68.5) (width 0.25) (layer F.Cu) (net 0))
 (segment (start 182.615 66.04) (end 184.15 67.575) (width 0.25) (layer F.Cu) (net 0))
 (segment (start 176.45 66.04) (end 182.615 66.04) (width 0.25) (layer F.Cu) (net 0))
 (segment (start 184.15 67.575) (end 193.04 67.575) (width 0.25) (layer F.Cu) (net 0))
 (segment (start 193.04 67.575) (end 201.93 67.575) (width 0.25) (layer F.Cu) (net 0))
 (segment (start 201.93 67.575) (end 210.82 67.575) (width 0.25) (layer F.Cu) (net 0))
 (segment (start 210.82 67.575) (end 219.71 67.575) (width 0.25) (layer F.Cu) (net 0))
 (segment (start 219.71 67.575) (end 228.6 67.575) (width 0.25) (layer F.Cu) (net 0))
 (segment (start 228.6 67.575) (end 237.49 67.575) (width 0.25) (layer F.Cu) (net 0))
 (segment (start 237.49 67.575) (end 246.38 67.575) (width 0.25) (layer F.Cu) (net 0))
 (segment (start 181.875 69.85) (end 184.15 72.125) (width 0.25) (layer F.Cu) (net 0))
 (segment (start 176.53 69.85) (end 181.875 69.85) (width 0.25) (layer F.Cu) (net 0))
 (segment (start 184.15 72.125) (end 193.04 72.125) (width 0.25) (layer F.Cu) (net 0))
 (segment (start 193.04 72.125) (end 201.93 72.125) (width 0.25) (layer F.Cu) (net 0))
 (segment (start 201.93 72.125) (end 210.82 72.125) (width 0.25) (layer F.Cu) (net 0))
 (segment (start 210.82 72.125) (end 219.71 72.125) (width 0.25) (layer F.Cu) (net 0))
 (segment (start 219.71 72.125) (end 228.6 72.125) (width 0.25) (layer F.Cu) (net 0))
 (segment (start 228.6 72.125) (end 237.49 72.125) (width 0.25) (layer F.Cu) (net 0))
 (segment (start 237.49 72.125) (end 246.38 72.125) (width 0.25) (layer F.Cu) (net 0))
 (segment (start 246.38 72.125) (end 248.655 69.85) (width 0.25) (layer F.Cu) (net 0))
 (segment (start 247.30071 60.34571) (end 246.38 59.425) (width 0.25) (layer F.Cu) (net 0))
 (segment (start 248.655 61.7) (end 247.30071 60.34571) (width 0.25) (layer F.Cu) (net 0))
 (segment (start 248.655 69.85) (end 248.655 61.7) (width 0.25) (layer F.Cu) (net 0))
 (segment (start 95.25 67.575) (end 95.25 64.77) (width 0.25) (layer F.Cu) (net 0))
 (segment (start 95.25 64.77) (end 92.71 62.23) (width 0.25) (layer F.Cu) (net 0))
 (segment (start 92.71 49.265) (end 95.25 46.725) (width 0.25) (layer F.Cu) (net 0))
 (segment (start 92.975 54.875) (end 95.25 54.875) (width 0.25) (layer F.Cu) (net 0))
 (segment (start 92.71 54.61) (end 92.975 54.875) (width 0.25) (layer F.Cu) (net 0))
 (segment (start 92.71 54.61) (end 92.71 49.265) (width 0.25) (layer F.Cu) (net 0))
 (segment (start 92.71 62.23) (end 92.71 54.61) (width 0.25) (layer F.Cu) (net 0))
 (segment (start 95.25 72.125) (end 93.715 72.125) (width 0.25) (layer F.Cu) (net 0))
 (segment (start 93.715 72.125) (end 91.44 69.85) (width 0.25) (layer F.Cu) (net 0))
 (segment (start 91.44 69.85) (end 91.44 44.45) (width 0.25) (layer F.Cu) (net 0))
 (segment (start 93.715 42.175) (end 95.25 42.175) (width 0.25) (layer F.Cu) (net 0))
 (segment (start 91.44 44.45) (end 93.715 42.175) (width 0.25) (layer F.Cu) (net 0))
 (segment (start 95.25 54.875) (end 104.14 54.875) (width 0.25) (layer F.Cu) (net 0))
 (segment (start 95.25 59.425) (end 104.14 59.425) (width 0.25) (layer F.Cu) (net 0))
 (segment (start 95.25 46.725) (end 104.14 46.725) (width 0.25) (layer F.Cu) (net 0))
 (segment (start 95.25 42.175) (end 104.14 42.175) (width 0.25) (layer F.Cu) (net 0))
 (segment (start 104.14 42.175) (end 113.03 42.175) (width 0.25) (layer F.Cu) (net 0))
 (segment (start 113.03 42.175) (end 121.92 42.175) (width 0.25) (layer F.Cu) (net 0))
 (segment (start 121.92 42.175) (end 130.81 42.175) (width 0.25) (layer F.Cu) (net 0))
 (segment (start 130.81 42.175) (end 139.7 42.175) (width 0.25) (layer F.Cu) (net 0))
 (segment (start 139.7 42.175) (end 148.59 42.175) (width 0.25) (layer F.Cu) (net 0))
 (segment (start 148.59 42.175) (end 157.48 42.175) (width 0.25) (layer F.Cu) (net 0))
 (segment (start 157.48 42.175) (end 166.37 42.175) (width 0.25) (layer F.Cu) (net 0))
 (segment (start 166.37 42.175) (end 175.26 42.175) (width 0.25) (layer F.Cu) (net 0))
 (segment (start 175.26 42.175) (end 184.15 42.175) (width 0.25) (layer F.Cu) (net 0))
 (segment (start 184.15 42.175) (end 193.04 42.175) (width 0.25) (layer F.Cu) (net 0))
 (segment (start 193.04 42.175) (end 201.93 42.175) (width 0.25) (layer F.Cu) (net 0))
 (segment (start 201.93 42.175) (end 210.82 42.175) (width 0.25) (layer F.Cu) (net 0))
 (segment (start 210.82 42.175) (end 219.71 42.175) (width 0.25) (layer F.Cu) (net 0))
 (segment (start 219.71 42.175) (end 228.6 42.175) (width 0.25) (layer F.Cu) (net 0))
 (segment (start 228.6 42.175) (end 237.49 42.175) (width 0.25) (layer F.Cu) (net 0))
 (segment (start 237.49 42.175) (end 246.38 42.175) (width 0.25) (layer F.Cu) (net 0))
 (segment (start 246.38 46.725) (end 237.49 46.725) (width 0.25) (layer F.Cu) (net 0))
 (segment (start 246.38 59.425) (end 248.655 57.15) (width 0.25) (layer F.Cu) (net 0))
 (segment (start 248.655 44.45) (end 246.38 42.175) (width 0.25) (layer F.Cu) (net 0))
 (segment (start 248.655 57.15) (end 248.655 44.45) (width 0.25) (layer F.Cu) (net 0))
 (segment (start 246.38 54.875) (end 237.49 54.875) (width 0.25) (layer F.Cu) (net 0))
 (segment (start 237.49 54.875) (end 228.6 54.875) (width 0.25) (layer F.Cu) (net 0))
 (segment (start 219.71 54.875) (end 228.6 54.875) (width 0.25) (layer F.Cu) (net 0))
 (segment (start 210.82 54.875) (end 219.71 54.875) (width 0.25) (layer F.Cu) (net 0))
 (segment (start 201.93 54.875) (end 210.82 54.875) (width 0.25) (layer F.Cu) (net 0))
 (segment (start 193.04 54.875) (end 201.93 54.875) (width 0.25) (layer F.Cu) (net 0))
 (segment (start 184.15 54.875) (end 193.04 54.875) (width 0.25) (layer F.Cu) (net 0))
 (segment (start 184.15 59.425) (end 193.04 59.425) (width 0.25) (layer F.Cu) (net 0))
 (segment (start 201.93 59.425) (end 193.04 59.425) (width 0.25) (layer F.Cu) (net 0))
 (segment (start 201.93 59.425) (end 210.82 59.425) (width 0.25) (layer F.Cu) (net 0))
 (segment (start 210.82 59.425) (end 219.71 59.425) (width 0.25) (layer F.Cu) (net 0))
 (segment (start 219.71 59.425) (end 228.6 59.425) (width 0.25) (layer F.Cu) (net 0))
 (segment (start 228.6 59.425) (end 237.49 59.425) (width 0.25) (layer F.Cu) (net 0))
 (segment (start 237.49 59.425) (end 246.38 59.425) (width 0.25) (layer F.Cu) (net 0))
 (segment (start 184.15 46.725) (end 193.04 46.725) (width 0.25) (layer F.Cu) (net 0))
 (segment (start 193.04 46.725) (end 201.93 46.725) (width 0.25) (layer F.Cu) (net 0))
 (segment (start 201.93 46.725) (end 210.82 46.725) (width 0.25) (layer F.Cu) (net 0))
 (segment (start 210.82 46.725) (end 219.71 46.725) (width 0.25) (layer F.Cu) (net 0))
 (segment (start 219.71 46.725) (end 228.6 46.725) (width 0.25) (layer F.Cu) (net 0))
 (segment (start 228.6 46.725) (end 237.49 46.725) (width 0.25) (layer F.Cu) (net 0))
 (segment (start 104.14 46.725) (end 113.03 46.725) (width 0.25) (layer F.Cu) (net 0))
 (segment (start 113.03 46.725) (end 121.92 46.725) (width 0.25) (layer F.Cu) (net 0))
 (segment (start 121.92 46.725) (end 130.81 46.725) (width 0.25) (layer F.Cu) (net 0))
 (segment (start 130.81 46.725) (end 139.7 46.725) (width 0.25) (layer F.Cu) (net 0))
 (segment (start 139.7 46.725) (end 148.59 46.725) (width 0.25) (layer F.Cu) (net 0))
 (segment (start 148.59 46.725) (end 157.48 46.725) (width 0.25) (layer F.Cu) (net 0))
 (segment (start 157.48 46.725) (end 166.37 46.725) (width 0.25) (layer F.Cu) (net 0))
 (segment (start 166.37 46.725) (end 175.26 46.725) (width 0.25) (layer F.Cu) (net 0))
 (segment (start 175.26 46.725) (end 184.15 46.725) (width 0.25) (layer F.Cu) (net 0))
 (segment (start 184.15 54.875) (end 175.26 54.875) (width 0.25) (layer F.Cu) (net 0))
 (segment (start 175.26 54.875) (end 166.37 54.875) (width 0.25) (layer F.Cu) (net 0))
 (segment (start 166.37 54.875) (end 157.48 54.875) (width 0.25) (layer F.Cu) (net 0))
 (segment (start 157.48 54.875) (end 148.59 54.875) (width 0.25) (layer F.Cu) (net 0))
 (segment (start 148.59 54.875) (end 139.7 54.875) (width 0.25) (layer F.Cu) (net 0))
 (segment (start 139.7 54.875) (end 130.81 54.875) (width 0.25) (layer F.Cu) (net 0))
 (segment (start 121.92 54.875) (end 130.81 54.875) (width 0.25) (layer F.Cu) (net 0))
 (segment (start 113.03 54.875) (end 121.92 54.875) (width 0.25) (layer F.Cu) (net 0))
 (segment (start 104.14 54.875) (end 113.03 54.875) (width 0.25) (layer F.Cu) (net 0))
 (segment (start 104.14 59.425) (end 113.03 59.425) (width 0.25) (layer F.Cu) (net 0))
 (segment (start 113.03 59.425) (end 121.92 59.425) (width 0.25) (layer F.Cu) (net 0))
 (segment (start 121.92 59.425) (end 130.81 59.425) (width 0.25) (layer F.Cu) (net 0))
 (segment (start 130.81 59.425) (end 139.7 59.425) (width 0.25) (layer F.Cu) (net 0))
 (segment (start 139.7 59.425) (end 149.595 59.425) (width 0.25) (layer F.Cu) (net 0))
 (segment (start 149.595 59.425) (end 148.59 59.425) (width 0.25) (layer F.Cu) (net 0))
 (segment (start 148.59 59.425) (end 157.48 59.425) (width 0.25) (layer F.Cu) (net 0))
 (segment (start 157.48 59.425) (end 166.37 59.425) (width 0.25) (layer F.Cu) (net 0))
 (segment (start 166.37 59.425) (end 175.26 59.425) (width 0.25) (layer F.Cu) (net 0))
 (segment (start 175.26 59.425) (end 184.15 59.425) (width 0.25) (layer F.Cu) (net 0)))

